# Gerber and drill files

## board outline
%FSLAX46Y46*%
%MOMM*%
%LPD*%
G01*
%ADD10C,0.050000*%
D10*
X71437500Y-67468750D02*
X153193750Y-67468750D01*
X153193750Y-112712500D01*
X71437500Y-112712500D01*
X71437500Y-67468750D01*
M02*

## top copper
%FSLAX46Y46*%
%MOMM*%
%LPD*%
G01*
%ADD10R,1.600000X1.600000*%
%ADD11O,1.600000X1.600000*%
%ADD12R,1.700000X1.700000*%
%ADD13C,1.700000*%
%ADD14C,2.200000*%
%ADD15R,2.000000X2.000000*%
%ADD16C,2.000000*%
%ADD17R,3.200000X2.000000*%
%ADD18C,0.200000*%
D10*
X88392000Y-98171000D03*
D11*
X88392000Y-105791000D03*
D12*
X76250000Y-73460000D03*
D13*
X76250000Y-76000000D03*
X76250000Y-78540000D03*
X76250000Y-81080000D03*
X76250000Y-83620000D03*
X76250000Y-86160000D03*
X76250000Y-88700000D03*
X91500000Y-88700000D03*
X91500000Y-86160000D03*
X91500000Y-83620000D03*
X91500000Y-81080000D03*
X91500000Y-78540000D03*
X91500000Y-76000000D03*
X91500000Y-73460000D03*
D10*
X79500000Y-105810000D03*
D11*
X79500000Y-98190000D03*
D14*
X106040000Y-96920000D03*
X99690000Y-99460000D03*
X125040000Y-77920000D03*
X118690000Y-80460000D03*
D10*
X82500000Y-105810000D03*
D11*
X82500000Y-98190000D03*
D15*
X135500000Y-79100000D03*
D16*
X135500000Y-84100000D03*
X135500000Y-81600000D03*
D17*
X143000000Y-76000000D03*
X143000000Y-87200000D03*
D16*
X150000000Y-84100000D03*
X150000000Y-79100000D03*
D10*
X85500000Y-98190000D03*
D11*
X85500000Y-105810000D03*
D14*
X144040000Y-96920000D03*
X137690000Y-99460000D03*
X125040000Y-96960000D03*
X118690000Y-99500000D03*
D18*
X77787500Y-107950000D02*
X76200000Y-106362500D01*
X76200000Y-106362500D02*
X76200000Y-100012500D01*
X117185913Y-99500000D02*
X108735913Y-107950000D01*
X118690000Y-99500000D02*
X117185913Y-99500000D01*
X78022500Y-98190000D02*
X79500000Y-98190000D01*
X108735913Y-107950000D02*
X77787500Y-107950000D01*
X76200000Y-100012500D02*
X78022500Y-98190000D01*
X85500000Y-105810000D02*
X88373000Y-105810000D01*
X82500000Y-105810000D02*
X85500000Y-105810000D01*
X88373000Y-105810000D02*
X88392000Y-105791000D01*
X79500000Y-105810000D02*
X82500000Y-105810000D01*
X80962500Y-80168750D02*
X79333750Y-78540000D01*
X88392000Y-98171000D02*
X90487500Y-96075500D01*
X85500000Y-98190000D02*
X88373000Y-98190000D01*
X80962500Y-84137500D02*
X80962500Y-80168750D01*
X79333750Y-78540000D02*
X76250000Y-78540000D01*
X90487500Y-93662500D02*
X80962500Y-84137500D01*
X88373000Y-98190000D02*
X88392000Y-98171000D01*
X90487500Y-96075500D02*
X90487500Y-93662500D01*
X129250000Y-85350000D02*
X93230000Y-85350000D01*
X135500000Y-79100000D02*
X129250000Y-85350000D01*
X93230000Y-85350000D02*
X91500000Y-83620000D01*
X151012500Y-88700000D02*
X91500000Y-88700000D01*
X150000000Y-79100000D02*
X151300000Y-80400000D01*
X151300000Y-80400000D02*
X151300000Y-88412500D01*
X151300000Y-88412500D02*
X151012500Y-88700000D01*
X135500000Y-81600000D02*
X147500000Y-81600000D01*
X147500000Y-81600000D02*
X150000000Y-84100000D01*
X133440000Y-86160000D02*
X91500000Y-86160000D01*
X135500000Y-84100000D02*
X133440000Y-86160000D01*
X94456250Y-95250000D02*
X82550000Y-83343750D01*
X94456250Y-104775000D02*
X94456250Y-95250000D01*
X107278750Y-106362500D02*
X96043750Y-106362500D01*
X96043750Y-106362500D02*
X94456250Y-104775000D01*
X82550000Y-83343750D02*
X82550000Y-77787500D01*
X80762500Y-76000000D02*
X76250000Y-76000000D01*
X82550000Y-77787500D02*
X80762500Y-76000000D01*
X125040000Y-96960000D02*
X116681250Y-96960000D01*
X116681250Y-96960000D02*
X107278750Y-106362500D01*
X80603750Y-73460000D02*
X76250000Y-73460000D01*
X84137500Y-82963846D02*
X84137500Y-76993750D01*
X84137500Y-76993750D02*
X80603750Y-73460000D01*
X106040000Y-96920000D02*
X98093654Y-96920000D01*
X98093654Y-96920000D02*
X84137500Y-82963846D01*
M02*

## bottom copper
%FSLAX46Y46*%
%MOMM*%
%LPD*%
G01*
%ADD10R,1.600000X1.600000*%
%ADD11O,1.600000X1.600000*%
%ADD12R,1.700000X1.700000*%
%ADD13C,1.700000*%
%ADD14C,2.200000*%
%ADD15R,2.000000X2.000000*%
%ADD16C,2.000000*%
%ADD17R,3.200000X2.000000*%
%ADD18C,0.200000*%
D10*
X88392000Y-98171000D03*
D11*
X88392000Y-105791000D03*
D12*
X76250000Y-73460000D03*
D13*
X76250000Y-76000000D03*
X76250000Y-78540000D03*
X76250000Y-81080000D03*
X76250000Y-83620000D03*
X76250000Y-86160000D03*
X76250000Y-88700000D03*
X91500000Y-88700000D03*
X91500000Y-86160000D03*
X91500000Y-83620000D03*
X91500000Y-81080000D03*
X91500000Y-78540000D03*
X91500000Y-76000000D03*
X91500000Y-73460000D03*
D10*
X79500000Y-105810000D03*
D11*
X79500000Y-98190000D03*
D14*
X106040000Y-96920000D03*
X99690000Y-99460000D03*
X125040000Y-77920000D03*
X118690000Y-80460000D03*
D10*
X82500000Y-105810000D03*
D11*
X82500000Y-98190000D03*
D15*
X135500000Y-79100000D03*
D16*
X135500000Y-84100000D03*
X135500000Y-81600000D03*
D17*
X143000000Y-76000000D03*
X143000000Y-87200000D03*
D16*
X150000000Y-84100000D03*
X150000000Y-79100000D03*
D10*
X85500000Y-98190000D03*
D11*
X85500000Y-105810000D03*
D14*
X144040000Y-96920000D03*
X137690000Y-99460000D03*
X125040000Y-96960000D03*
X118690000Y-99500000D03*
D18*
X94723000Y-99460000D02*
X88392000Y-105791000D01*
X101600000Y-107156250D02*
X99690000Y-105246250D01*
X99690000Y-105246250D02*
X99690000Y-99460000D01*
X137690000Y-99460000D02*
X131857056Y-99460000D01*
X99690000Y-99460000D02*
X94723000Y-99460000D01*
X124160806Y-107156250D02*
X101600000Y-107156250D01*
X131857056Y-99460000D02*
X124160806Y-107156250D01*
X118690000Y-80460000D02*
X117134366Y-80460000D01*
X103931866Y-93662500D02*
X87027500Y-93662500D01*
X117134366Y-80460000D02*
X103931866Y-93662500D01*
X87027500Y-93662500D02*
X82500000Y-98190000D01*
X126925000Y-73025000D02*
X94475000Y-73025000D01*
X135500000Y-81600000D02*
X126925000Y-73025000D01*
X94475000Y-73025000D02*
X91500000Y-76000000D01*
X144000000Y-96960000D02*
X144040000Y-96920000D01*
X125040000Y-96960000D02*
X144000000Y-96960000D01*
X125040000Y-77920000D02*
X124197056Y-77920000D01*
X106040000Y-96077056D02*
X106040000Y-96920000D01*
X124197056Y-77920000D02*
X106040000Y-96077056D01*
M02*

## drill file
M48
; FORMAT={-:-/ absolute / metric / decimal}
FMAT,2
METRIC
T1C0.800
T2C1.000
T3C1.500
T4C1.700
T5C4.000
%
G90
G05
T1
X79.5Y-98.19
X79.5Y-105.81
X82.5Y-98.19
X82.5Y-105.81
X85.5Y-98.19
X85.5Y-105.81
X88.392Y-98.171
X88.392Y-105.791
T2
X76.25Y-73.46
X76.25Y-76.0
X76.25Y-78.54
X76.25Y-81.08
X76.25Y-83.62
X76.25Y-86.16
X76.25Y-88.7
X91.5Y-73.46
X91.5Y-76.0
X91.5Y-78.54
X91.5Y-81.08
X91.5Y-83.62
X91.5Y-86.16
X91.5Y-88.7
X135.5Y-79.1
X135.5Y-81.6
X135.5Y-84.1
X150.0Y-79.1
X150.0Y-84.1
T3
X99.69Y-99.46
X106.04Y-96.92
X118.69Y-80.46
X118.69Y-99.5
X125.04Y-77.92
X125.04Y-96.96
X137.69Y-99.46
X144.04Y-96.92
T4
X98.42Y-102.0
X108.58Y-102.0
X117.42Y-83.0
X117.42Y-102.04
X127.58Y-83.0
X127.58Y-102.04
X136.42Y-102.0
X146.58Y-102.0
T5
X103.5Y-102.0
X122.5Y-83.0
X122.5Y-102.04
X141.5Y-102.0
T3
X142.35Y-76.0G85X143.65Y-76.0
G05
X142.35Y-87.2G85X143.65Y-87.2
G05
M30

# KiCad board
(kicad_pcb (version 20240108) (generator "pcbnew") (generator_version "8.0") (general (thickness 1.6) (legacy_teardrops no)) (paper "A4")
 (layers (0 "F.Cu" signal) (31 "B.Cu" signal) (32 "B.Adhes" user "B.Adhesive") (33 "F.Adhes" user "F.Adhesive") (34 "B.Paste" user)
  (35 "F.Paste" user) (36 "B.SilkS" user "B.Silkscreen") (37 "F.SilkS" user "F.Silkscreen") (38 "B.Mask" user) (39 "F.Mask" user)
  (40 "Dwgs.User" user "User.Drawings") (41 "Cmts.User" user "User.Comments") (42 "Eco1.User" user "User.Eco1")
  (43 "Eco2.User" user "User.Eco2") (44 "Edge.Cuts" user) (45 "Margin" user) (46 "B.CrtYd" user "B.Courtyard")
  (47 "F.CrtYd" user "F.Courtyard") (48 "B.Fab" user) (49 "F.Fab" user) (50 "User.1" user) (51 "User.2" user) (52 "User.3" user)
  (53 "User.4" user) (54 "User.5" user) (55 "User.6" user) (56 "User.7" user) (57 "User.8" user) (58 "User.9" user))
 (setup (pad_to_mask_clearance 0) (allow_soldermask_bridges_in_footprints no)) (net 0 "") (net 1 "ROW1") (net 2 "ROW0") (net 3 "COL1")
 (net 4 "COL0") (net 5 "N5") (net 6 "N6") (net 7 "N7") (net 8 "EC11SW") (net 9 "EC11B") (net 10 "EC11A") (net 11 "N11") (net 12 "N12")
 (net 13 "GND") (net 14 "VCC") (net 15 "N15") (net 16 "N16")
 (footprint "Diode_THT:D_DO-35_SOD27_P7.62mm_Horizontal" (layer "F.Cu") (at 88.392 98.171 -90)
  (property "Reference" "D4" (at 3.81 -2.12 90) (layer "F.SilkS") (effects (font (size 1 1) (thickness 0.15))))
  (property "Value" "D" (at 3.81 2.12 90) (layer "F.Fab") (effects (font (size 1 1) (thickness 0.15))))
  (pad "1" thru_hole rect (at 0 0 270) (size 1.6 1.6) (drill 0.8) (layers "*.Cu" "*.Mask") (remove_unused_layers no) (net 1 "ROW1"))
  (pad "2" thru_hole oval (at 7.62 0 270) (size 1.6 1.6) (drill 0.8) (layers "*.Cu" "*.Mask") (remove_unused_layers no) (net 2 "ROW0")))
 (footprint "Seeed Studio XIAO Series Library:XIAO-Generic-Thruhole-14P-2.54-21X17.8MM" (layer "F.Cu") (at 83.875 81.08)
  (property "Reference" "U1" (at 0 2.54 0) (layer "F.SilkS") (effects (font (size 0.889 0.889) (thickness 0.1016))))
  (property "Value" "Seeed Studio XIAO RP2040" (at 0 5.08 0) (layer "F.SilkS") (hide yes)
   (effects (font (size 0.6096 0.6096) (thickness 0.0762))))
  (pad "1" thru_hole rect (at -7.625 -7.62) (size 1.7 1.7) (drill 1) (layers "*.Cu" "*.Mask") (remove_unused_layers no) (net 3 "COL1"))
  (pad "2" thru_hole circle (at -7.625 -5.08) (size 1.7 1.7) (drill 1) (layers "*.Cu" "*.Mask") (remove_unused_layers no) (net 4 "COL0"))
  (pad "3" thru_hole circle (at -7.625 -2.54) (size 1.7 1.7) (drill 1) (layers "*.Cu" "*.Mask") (remove_unused_layers no) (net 1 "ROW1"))
  (pad "4" thru_hole circle (at -7.625 0) (size 1.7 1.7) (drill 1) (layers "*.Cu" "*.Mask") (remove_unused_layers no) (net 2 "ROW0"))
  (pad "5" thru_hole circle (at -7.625 2.54) (size 1.7 1.7) (drill 1) (layers "*.Cu" "*.Mask") (remove_unused_layers no) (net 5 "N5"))
  (pad "6" thru_hole circle (at -7.625 5.08 180) (size 1.7 1.7) (drill 1) (layers "*.Cu" "*.Mask") (remove_unused_layers no) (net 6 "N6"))
  (pad "7" thru_hole circle (at -7.625 7.62) (size 1.7 1.7) (drill 1) (layers "*.Cu" "*.Mask") (remove_unused_layers no) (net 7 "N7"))
  (pad "8" thru_hole circle (at 7.625 7.62) (size 1.7 1.7) (drill 1) (layers "*.Cu" "*.Mask") (remove_unused_layers no) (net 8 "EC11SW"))
  (pad "9" thru_hole circle (at 7.625 5.08) (size 1.7 1.7) (drill 1) (layers "*.Cu" "*.Mask") (remove_unused_layers no) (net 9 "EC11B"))
  (pad "10" thru_hole circle (at 7.625 2.54) (size 1.7 1.7) (drill 1) (layers "*.Cu" "*.Mask") (remove_unused_layers no) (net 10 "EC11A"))
  (pad "11" thru_hole circle (at 7.625 0) (size 1.7 1.7) (drill 1) (layers "*.Cu" "*.Mask") (remove_unused_layers no) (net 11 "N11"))
  (pad "12" thru_hole circle (at 7.625 -2.54) (size 1.7 1.7) (drill 1) (layers "*.Cu" "*.Mask") (remove_unused_layers no) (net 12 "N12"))
  (pad "13" thru_hole circle (at 7.625 -5.08) (size 1.7 1.7) (drill 1) (layers "*.Cu" "*.Mask") (remove_unused_layers no) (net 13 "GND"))
  (pad "14" thru_hole circle (at 7.625 -7.62) (size 1.7 1.7) (drill 1) (layers "*.Cu" "*.Mask") (remove_unused_layers no) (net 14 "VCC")))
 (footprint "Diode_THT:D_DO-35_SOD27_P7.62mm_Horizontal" (layer "F.Cu") (at 79.5 105.81 90)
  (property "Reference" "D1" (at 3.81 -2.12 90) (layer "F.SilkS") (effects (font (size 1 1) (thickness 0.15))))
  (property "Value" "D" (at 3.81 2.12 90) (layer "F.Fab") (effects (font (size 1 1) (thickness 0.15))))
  (pad "1" thru_hole rect (at 0 0 90) (size 1.6 1.6) (drill 0.8) (layers "*.Cu" "*.Mask") (remove_unused_layers no) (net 2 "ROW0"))
  (pad "2" thru_hole oval (at 7.62 0 90) (size 1.6 1.6) (drill 0.8) (layers "*.Cu" "*.Mask") (remove_unused_layers no) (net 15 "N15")))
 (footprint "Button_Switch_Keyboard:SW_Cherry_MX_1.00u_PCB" (layer "F.Cu") (at 106.04 96.92)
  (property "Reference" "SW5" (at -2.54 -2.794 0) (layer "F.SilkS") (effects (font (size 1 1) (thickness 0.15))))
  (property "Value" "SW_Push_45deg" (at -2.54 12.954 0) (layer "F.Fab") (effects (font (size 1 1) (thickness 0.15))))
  (pad "" np_thru_hole circle (at -7.62 5.08) (size 1.7 1.7) (drill 1.7) (layers "*.Cu" "*.Mask"))
  (pad "" np_thru_hole circle (at -2.54 5.08) (size 4 4) (drill 4) (layers "*.Cu" "*.Mask"))
  (pad "" np_thru_hole circle (at 2.54 5.08) (size 1.7 1.7) (drill 1.7) (layers "*.Cu" "*.Mask"))
  (pad "1" thru_hole circle (at 0 0) (size 2.2 2.2) (drill 1.5) (layers "*.Cu" "*.Mask") (remove_unused_layers no) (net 3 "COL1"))
  (pad "2" thru_hole circle (at -6.35 2.54) (size 2.2 2.2) (drill 1.5) (layers "*.Cu" "*.Mask") (remove_unused_layers no) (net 2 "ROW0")))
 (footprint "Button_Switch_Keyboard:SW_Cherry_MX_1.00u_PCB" (layer "F.Cu") (at 125.04 77.92)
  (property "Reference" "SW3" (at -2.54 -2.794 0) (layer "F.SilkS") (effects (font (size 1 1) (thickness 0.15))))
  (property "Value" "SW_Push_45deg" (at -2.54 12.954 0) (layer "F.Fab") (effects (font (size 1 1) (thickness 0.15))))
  (pad "" np_thru_hole circle (at -7.62 5.08) (size 1.7 1.7) (drill 1.7) (layers "*.Cu" "*.Mask"))
  (pad "" np_thru_hole circle (at -2.54 5.08) (size 4 4) (drill 4) (layers "*.Cu" "*.Mask"))
  (pad "" np_thru_hole circle (at 2.54 5.08) (size 1.7 1.7) (drill 1.7) (layers "*.Cu" "*.Mask"))
  (pad "1" thru_hole circle (at 0 0) (size 2.2 2.2) (drill 1.5) (layers "*.Cu" "*.Mask") (remove_unused_layers no) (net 3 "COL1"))
  (pad "2" thru_hole circle (at -6.35 2.54) (size 2.2 2.2) (drill 1.5) (layers "*.Cu" "*.Mask") (remove_unused_layers no) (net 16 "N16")))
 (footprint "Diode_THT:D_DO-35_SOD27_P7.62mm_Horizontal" (layer "F.Cu") (at 82.5 105.81 90)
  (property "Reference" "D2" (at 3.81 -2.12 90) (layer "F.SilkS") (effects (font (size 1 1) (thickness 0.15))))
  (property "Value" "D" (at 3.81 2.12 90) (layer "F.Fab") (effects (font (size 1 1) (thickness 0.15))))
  (pad "1" thru_hole rect (at 0 0 90) (size 1.6 1.6) (drill 0.8) (layers "*.Cu" "*.Mask") (remove_unused_layers no) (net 2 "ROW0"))
  (pad "2" thru_hole oval (at 7.62 0 90) (size 1.6 1.6) (drill 0.8) (layers "*.Cu" "*.Mask") (remove_unused_layers no) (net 16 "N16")))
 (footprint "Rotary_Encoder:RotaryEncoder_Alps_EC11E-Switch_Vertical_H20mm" (layer "F.Cu") (at 135.5 79.1)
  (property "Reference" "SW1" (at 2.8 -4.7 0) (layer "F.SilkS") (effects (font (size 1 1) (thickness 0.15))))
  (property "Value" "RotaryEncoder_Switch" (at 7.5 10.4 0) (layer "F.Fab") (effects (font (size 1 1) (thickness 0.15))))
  (pad "A" thru_hole rect (at 0 0) (size 2 2) (drill 1) (layers "*.Cu" "*.Mask") (remove_unused_layers no) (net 10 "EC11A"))
  (pad "B" thru_hole circle (at 0 5) (size 2 2) (drill 1) (layers "*.Cu" "*.Mask") (remove_unused_layers no) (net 9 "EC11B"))
  (pad "C" thru_hole circle (at 0 2.5) (size 2 2) (drill 1) (layers "*.Cu" "*.Mask") (remove_unused_layers no) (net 13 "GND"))
  (pad "MP" thru_hole rect (at 7.5 -3.1) (size 3.2 2) (drill oval 2.8 1.5) (layers "*.Cu" "*.Mask") (remove_unused_layers no))
  (pad "MP" thru_hole rect (at 7.5 8.1) (size 3.2 2) (drill oval 2.8 1.5) (layers "*.Cu" "*.Mask") (remove_unused_layers no))
  (pad "S1" thru_hole circle (at 14.5 5) (size 2 2) (drill 1) (layers "*.Cu" "*.Mask") (remove_unused_layers no) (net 13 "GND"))
  (pad "S2" thru_hole circle (at 14.5 0) (size 2 2) (drill 1) (layers "*.Cu" "*.Mask") (remove_unused_layers no) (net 8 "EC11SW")))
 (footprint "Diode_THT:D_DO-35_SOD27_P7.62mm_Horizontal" (layer "F.Cu") (at 85.5 98.19 -90)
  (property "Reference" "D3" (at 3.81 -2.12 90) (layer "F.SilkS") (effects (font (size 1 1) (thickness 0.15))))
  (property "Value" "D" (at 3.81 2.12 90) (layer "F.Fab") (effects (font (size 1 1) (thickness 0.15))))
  (pad "1" thru_hole rect (at 0 0 270) (size 1.6 1.6) (drill 0.8) (layers "*.Cu" "*.Mask") (remove_unused_layers no) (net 1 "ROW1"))
  (pad "2" thru_hole oval (at 7.62 0 270) (size 1.6 1.6) (drill 0.8) (layers "*.Cu" "*.Mask") (remove_unused_layers no) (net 2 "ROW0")))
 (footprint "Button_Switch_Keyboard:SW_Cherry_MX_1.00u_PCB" (layer "F.Cu") (at 144.04 96.92)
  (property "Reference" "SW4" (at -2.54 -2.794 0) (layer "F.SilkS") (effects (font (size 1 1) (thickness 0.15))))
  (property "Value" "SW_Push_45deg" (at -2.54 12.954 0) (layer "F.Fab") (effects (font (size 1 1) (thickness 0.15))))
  (pad "" np_thru_hole circle (at -7.62 5.08) (size 1.7 1.7) (drill 1.7) (layers "*.Cu" "*.Mask"))
  (pad "" np_thru_hole circle (at -2.54 5.08) (size 4 4) (drill 4) (layers "*.Cu" "*.Mask"))
  (pad "" np_thru_hole circle (at 2.54 5.08) (size 1.7 1.7) (drill 1.7) (layers "*.Cu" "*.Mask"))
  (pad "1" thru_hole circle (at 0 0) (size 2.2 2.2) (drill 1.5) (layers "*.Cu" "*.Mask") (remove_unused_layers no) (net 4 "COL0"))
  (pad "2" thru_hole circle (at -6.35 2.54) (size 2.2 2.2) (drill 1.5) (layers "*.Cu" "*.Mask") (remove_unused_layers no) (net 2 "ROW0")))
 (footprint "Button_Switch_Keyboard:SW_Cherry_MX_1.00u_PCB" (layer "F.Cu") (at 125.04 96.96)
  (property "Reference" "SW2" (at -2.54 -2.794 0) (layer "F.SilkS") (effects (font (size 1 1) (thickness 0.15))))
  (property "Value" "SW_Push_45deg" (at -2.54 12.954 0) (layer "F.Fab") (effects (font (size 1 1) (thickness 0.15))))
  (pad "" np_thru_hole circle (at -7.62 5.08) (size 1.7 1.7) (drill 1.7) (layers "*.Cu" "*.Mask"))
  (pad "" np_thru_hole circle (at -2.54 5.08) (size 4 4) (drill 4) (layers "*.Cu" "*.Mask"))
  (pad "" np_thru_hole circle (at 2.54 5.08) (size 1.7 1.7) (drill 1.7) (layers "*.Cu" "*.Mask"))
  (pad "1" thru_hole circle (at 0 0) (size 2.2 2.2) (drill 1.5) (layers "*.Cu" "*.Mask") (remove_unused_layers no) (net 4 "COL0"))
  (pad "2" thru_hole circle (at -6.35 2.54) (size 2.2 2.2) (drill 1.5) (layers "*.Cu" "*.Mask") (remove_unused_layers no) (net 15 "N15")))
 (gr_rect (start 71.4375 67.46875) (end 153.19375 112.7125) (stroke (width 0.05) (type default)) (fill none) (layer "Edge.Cuts"))
 (segment (start 77.7875 107.95) (end 76.2 106.3625) (width 0.2) (layer "F.Cu") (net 15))
 (segment (start 76.2 106.3625) (end 76.2 100.0125) (width 0.2) (layer "F.Cu") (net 15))
 (segment (start 117.185913 99.5) (end 108.735913 107.95) (width 0.2) (layer "F.Cu") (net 15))
 (segment (start 118.69 99.5) (end 117.185913 99.5) (width 0.2) (layer "F.Cu") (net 15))
 (segment (start 78.0225 98.19) (end 79.5 98.19) (width 0.2) (layer "F.Cu") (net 15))
 (segment (start 108.735913 107.95) (end 77.7875 107.95) (width 0.2) (layer "F.Cu") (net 15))
 (segment (start 76.2 100.0125) (end 78.0225 98.19) (width 0.2) (layer "F.Cu") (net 15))
 (segment (start 85.5 105.81) (end 88.373 105.81) (width 0.2) (layer "F.Cu") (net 2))
 (segment (start 82.5 105.81) (end 85.5 105.81) (width 0.2) (layer "F.Cu") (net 2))
 (segment (start 88.373 105.81) (end 88.392 105.791) (width 0.2) (layer "F.Cu") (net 2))
 (segment (start 79.5 105.81) (end 82.5 105.81) (width 0.2) (layer "F.Cu") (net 2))
 (segment (start 94.723 99.46) (end 88.392 105.791) (width 0.2) (layer "B.Cu") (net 2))
 (segment (start 101.6 107.15625) (end 99.69 105.24625) (width 0.2) (layer "B.Cu") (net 2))
 (segment (start 99.69 105.24625) (end 99.69 99.46) (width 0.2) (layer "B.Cu") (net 2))
 (segment (start 137.69 99.46) (end 131.857056 99.46) (width 0.2) (layer "B.Cu") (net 2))
 (segment (start 99.69 99.46) (end 94.723 99.46) (width 0.2) (layer "B.Cu") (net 2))
 (segment (start 124.160806 107.15625) (end 101.6 107.15625) (width 0.2) (layer "B.Cu") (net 2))
 (segment (start 131.857056 99.46) (end 124.160806 107.15625) (width 0.2) (layer "B.Cu") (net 2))
 (segment (start 118.69 80.46) (end 117.134366 80.46) (width 0.2) (layer "B.Cu") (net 16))
 (segment (start 103.931866 93.6625) (end 87.0275 93.6625) (width 0.2) (layer "B.Cu") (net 16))
 (segment (start 117.134366 80.46) (end 103.931866 93.6625) (width 0.2) (layer "B.Cu") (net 16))
 (segment (start 87.0275 93.6625) (end 82.5 98.19) (width 0.2) (layer "B.Cu") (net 16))
 (segment (start 80.9625 80.16875) (end 79.33375 78.54) (width 0.2) (layer "F.Cu") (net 1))
 (segment (start 88.392 98.171) (end 90.4875 96.0755) (width 0.2) (layer "F.Cu") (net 1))
 (segment (start 85.5 98.19) (end 88.373 98.19) (width 0.2) (layer "F.Cu") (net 1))
 (segment (start 80.9625 84.1375) (end 80.9625 80.16875) (width 0.2) (layer "F.Cu") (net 1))
 (segment (start 79.33375 78.54) (end 76.25 78.54) (width 0.2) (layer "F.Cu") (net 1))
 (segment (start 90.4875 93.6625) (end 80.9625 84.1375) (width 0.2) (layer "F.Cu") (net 1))
 (segment (start 88.373 98.19) (end 88.392 98.171) (width 0.2) (layer "F.Cu") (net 1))
 (segment (start 90.4875 96.0755) (end 90.4875 93.6625) (width 0.2) (layer "F.Cu") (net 1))
 (segment (start 129.25 85.35) (end 93.23 85.35) (width 0.2) (layer "F.Cu") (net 10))
 (segment (start 135.5 79.1) (end 129.25 85.35) (width 0.2) (layer "F.Cu") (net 10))
 (segment (start 93.23 85.35) (end 91.5 83.62) (width 0.2) (layer "F.Cu") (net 10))
 (segment (start 151.0125 88.7) (end 91.5 88.7) (width 0.2) (layer "F.Cu") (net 8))
 (segment (start 150 79.1) (end 151.3 80.4) (width 0.2) (layer "F.Cu") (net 8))
 (segment (start 151.3 80.4) (end 151.3 88.4125) (width 0.2) (layer "F.Cu") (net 8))
 (segment (start 151.3 88.4125) (end 151.0125 88.7) (width 0.2) (layer "F.Cu") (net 8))
 (segment (start 135.5 81.6) (end 147.5 81.6) (width 0.2) (layer "F.Cu") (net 13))
 (segment (start 147.5 81.6) (end 150 84.1) (width 0.2) (layer "F.Cu") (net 13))
 (segment (start 126.925 73.025) (end 94.475 73.025) (width 0.2) (layer "B.Cu") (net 13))
 (segment (start 135.5 81.6) (end 126.925 73.025) (width 0.2) (layer "B.Cu") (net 13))
 (segment (start 94.475 73.025) (end 91.5 76) (width 0.2) (layer "B.Cu") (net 13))
 (segment (start 133.44 86.16) (end 91.5 86.16) (width 0.2) (layer "F.Cu") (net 9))
 (segment (start 135.5 84.1) (end 133.44 86.16) (width 0.2) (layer "F.Cu") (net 9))
 (segment (start 94.45625 95.25) (end 82.55 83.34375) (width 0.2) (layer "F.Cu") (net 4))
 (segment (start 94.45625 104.775) (end 94.45625 95.25) (width 0.2) (layer "F.Cu") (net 4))
 (segment (start 107.27875 106.3625) (end 96.04375 106.3625) (width 0.2) (layer "F.Cu") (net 4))
 (segment (start 96.04375 106.3625) (end 94.45625 104.775) (width 0.2) (layer "F.Cu") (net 4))
 (segment (start 82.55 83.34375) (end 82.55 77.7875) (width 0.2) (layer "F.Cu") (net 4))
 (segment (start 80.7625 76) (end 76.25 76) (width 0.2) (layer "F.Cu") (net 4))
 (segment (start 82.55 77.7875) (end 80.7625 76) (width 0.2) (layer "F.Cu") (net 4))
 (segment (start 125.04 96.96) (end 116.68125 96.96) (width 0.2) (layer "F.Cu") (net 4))
 (segment (start 116.68125 96.96) (end 107.27875 106.3625) (width 0.2) (layer "F.Cu") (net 4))
 (segment (start 144 96.96) (end 144.04 96.92) (width 0.2) (layer "B.Cu") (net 4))
 (segment (start 125.04 96.96) (end 144 96.96) (width 0.2) (layer "B.Cu") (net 4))
 (segment (start 80.60375 73.46) (end 76.25 73.46) (width 0.2) (layer "F.Cu") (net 3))
 (segment (start 84.1375 82.963846) (end 84.1375 76.99375) (width 0.2) (layer "F.Cu") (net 3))
 (segment (start 84.1375 76.99375) (end 80.60375 73.46) (width 0.2) (layer "F.Cu") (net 3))
 (segment (start 106.04 96.92) (end 98.093654 96.92) (width 0.2) (layer "F.Cu") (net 3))
 (segment (start 98.093654 96.92) (end 84.1375 82.963846) (width 0.2) (layer "F.Cu") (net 3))
 (segment (start 125.04 77.92) (end 124.197056 77.92) (width 0.2) (layer "B.Cu") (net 3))
 (segment (start 106.04 96.077056) (end 106.04 96.92) (width 0.2) (layer "B.Cu") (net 3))
 (segment (start 124.197056 77.92) (end 106.04 96.077056) (width 0.2) (layer "B.Cu") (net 3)))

